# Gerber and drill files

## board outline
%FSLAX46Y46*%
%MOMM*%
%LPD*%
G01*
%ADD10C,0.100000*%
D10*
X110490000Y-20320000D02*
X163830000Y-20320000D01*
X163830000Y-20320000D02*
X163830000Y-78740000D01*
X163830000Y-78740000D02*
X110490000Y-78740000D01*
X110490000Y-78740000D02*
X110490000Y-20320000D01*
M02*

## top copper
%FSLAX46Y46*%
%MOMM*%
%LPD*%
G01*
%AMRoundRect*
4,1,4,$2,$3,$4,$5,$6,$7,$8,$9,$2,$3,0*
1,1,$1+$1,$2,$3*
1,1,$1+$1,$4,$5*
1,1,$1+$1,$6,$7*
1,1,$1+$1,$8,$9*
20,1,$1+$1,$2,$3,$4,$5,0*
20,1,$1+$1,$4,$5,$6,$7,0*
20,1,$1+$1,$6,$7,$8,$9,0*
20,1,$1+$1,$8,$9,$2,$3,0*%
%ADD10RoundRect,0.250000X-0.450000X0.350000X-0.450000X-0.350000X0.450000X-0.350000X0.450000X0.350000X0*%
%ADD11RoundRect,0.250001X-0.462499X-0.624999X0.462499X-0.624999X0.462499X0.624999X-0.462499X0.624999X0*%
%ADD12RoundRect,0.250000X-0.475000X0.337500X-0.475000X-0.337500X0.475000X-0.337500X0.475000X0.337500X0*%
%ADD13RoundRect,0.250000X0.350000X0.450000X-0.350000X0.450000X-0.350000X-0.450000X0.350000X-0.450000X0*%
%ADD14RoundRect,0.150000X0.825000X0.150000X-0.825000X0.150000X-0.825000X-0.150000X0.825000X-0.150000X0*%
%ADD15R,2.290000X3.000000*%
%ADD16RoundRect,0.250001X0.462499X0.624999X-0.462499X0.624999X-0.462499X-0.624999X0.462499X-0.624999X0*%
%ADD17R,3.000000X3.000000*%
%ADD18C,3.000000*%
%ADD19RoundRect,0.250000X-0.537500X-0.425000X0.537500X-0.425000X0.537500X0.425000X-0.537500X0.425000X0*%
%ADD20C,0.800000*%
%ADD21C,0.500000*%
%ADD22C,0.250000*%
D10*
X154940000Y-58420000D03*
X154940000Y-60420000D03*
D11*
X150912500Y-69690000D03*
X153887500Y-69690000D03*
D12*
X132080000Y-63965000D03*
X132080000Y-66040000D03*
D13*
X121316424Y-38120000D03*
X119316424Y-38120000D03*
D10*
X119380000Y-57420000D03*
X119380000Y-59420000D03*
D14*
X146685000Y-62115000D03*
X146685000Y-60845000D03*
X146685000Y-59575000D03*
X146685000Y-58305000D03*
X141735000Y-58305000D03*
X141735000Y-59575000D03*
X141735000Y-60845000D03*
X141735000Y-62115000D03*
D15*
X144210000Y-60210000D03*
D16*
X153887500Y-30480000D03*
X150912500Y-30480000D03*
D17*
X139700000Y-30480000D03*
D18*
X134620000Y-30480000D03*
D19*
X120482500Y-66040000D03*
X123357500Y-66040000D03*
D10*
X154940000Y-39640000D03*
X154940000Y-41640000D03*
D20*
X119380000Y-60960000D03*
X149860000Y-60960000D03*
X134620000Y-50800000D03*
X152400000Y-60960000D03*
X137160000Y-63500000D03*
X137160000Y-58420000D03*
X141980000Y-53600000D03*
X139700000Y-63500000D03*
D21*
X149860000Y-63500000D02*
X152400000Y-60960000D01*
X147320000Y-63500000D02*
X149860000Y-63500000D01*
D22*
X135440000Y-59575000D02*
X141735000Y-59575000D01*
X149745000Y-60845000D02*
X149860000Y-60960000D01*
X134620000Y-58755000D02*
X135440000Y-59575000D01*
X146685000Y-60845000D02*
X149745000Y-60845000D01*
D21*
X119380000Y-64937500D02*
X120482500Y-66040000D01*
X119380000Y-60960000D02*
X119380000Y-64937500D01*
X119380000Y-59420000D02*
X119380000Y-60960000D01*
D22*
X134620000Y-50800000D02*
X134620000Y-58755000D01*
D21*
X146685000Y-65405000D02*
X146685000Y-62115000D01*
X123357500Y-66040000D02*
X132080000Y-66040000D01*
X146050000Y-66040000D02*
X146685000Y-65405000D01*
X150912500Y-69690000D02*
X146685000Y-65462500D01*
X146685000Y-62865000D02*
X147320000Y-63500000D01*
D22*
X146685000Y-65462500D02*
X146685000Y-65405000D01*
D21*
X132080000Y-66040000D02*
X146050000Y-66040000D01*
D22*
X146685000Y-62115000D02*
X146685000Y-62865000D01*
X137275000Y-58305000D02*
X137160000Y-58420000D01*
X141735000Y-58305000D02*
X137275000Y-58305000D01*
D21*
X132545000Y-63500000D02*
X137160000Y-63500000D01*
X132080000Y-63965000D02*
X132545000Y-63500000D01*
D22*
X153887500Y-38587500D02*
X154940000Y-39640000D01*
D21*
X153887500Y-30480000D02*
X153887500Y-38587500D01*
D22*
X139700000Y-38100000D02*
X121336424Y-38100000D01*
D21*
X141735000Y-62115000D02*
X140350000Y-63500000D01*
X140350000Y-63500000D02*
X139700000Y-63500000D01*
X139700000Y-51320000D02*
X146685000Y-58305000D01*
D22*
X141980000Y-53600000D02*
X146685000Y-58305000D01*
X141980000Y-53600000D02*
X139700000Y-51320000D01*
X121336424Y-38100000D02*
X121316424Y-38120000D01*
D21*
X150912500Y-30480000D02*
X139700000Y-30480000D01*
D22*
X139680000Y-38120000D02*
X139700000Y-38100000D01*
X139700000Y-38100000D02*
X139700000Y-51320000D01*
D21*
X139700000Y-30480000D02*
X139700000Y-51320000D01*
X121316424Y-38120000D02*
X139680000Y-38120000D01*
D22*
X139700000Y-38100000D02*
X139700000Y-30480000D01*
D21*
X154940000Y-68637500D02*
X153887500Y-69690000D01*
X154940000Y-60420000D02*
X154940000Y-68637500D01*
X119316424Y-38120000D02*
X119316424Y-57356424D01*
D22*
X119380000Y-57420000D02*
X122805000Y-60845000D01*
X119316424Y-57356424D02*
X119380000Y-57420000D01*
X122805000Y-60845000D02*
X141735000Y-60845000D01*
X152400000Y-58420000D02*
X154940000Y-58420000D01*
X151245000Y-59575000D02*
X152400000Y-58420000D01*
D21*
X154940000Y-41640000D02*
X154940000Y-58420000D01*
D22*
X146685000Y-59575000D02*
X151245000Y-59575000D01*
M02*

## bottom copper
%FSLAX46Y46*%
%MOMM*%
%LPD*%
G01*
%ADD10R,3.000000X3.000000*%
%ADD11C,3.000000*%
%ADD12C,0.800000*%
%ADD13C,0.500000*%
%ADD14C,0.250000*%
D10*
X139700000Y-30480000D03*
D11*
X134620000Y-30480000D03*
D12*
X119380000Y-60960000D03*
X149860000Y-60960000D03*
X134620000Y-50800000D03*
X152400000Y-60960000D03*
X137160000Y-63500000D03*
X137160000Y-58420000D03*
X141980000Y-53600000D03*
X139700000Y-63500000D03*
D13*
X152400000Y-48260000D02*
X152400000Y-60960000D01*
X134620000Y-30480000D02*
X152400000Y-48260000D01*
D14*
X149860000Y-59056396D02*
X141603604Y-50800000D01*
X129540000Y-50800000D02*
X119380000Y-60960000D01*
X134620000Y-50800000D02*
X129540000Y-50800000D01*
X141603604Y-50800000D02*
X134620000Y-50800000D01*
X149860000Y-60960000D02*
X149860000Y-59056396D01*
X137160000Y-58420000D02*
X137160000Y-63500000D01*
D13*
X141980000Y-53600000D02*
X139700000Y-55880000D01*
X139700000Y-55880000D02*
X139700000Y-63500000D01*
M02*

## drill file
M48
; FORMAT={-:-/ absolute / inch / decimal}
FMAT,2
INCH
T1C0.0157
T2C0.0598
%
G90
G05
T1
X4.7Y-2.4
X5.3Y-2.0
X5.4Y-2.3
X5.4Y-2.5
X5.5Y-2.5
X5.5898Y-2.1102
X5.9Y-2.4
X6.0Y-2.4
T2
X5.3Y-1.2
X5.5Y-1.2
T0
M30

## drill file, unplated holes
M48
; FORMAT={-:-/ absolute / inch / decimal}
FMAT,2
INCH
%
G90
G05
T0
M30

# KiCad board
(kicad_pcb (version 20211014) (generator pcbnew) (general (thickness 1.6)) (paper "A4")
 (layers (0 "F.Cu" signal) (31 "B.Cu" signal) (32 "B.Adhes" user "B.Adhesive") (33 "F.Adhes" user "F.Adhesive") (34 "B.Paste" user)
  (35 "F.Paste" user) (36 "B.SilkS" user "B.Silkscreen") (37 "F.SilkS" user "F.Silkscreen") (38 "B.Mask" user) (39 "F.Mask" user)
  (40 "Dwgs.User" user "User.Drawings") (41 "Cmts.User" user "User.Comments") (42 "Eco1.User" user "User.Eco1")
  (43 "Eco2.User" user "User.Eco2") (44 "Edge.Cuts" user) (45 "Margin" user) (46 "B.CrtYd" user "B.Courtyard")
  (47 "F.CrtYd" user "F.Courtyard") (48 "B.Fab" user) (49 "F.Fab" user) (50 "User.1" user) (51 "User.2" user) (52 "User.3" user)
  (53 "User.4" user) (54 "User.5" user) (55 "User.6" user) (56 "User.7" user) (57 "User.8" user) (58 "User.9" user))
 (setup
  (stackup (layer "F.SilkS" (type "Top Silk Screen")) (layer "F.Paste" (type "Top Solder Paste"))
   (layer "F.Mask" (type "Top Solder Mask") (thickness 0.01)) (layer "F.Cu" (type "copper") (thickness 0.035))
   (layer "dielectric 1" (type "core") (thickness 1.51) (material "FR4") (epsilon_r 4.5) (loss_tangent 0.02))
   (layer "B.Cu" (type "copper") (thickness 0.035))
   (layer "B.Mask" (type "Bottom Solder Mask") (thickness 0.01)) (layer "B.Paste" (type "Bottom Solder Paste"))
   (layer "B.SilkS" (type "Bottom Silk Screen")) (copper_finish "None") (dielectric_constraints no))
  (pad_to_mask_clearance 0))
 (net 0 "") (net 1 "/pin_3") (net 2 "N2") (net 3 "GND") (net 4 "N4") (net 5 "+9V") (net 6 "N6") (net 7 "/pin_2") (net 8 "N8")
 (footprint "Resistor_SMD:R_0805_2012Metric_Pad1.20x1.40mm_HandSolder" (layer "F.Cu") (at 154.94 59.42 -90)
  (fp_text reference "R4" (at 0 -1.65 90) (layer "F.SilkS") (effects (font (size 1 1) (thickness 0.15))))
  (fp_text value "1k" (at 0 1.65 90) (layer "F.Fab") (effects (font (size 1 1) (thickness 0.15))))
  (pad "1" smd roundrect (at -1 0 270) (size 1.2 1.4) (layers "F.Cu" "F.Paste" "F.Mask") (roundrect_rratio 0.2083333333) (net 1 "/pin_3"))
  (pad "2" smd roundrect (at 1 0 270) (size 1.2 1.4) (layers "F.Cu" "F.Paste" "F.Mask") (roundrect_rratio 0.2083333333) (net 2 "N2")))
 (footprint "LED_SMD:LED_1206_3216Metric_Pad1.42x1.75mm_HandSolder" (layer "F.Cu") (at 152.4 69.69)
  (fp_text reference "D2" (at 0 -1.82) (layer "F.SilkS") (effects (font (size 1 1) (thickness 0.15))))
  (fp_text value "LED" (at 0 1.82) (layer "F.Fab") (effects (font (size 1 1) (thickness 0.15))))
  (pad "1" smd roundrect (at -1.4875 0) (size 1.425 1.75) (layers "F.Cu" "F.Paste" "F.Mask") (roundrect_rratio 0.1754392982) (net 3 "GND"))
  (pad "2" smd roundrect (at 1.4875 0) (size 1.425 1.75) (layers "F.Cu" "F.Paste" "F.Mask") (roundrect_rratio 0.1754392982) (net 2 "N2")))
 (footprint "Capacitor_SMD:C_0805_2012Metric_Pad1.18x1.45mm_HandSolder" (layer "F.Cu") (at 132.08 65.0025 -90)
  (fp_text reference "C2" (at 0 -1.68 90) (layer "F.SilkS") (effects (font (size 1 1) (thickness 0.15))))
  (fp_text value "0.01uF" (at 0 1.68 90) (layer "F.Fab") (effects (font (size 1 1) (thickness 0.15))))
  (pad "1" smd roundrect (at -1.0375 0 270) (size 1.175 1.45) (layers "F.Cu" "F.Paste" "F.Mask") (roundrect_rratio 0.2127659574)
   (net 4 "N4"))
  (pad "2" smd roundrect (at 1.0375 0 270) (size 1.175 1.45) (layers "F.Cu" "F.Paste" "F.Mask") (roundrect_rratio 0.2127659574)
   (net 3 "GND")))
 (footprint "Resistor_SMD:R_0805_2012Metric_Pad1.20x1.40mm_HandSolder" (layer "F.Cu") (at 120.316424 38.12 180)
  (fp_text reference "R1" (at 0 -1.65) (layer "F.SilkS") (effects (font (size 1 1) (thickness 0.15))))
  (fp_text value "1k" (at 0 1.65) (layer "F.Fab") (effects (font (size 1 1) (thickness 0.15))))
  (pad "1" smd roundrect (at -1 0 180) (size 1.2 1.4) (layers "F.Cu" "F.Paste" "F.Mask") (roundrect_rratio 0.2083333333) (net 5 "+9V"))
  (pad "2" smd roundrect (at 1 0 180) (size 1.2 1.4) (layers "F.Cu" "F.Paste" "F.Mask") (roundrect_rratio 0.2083333333) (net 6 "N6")))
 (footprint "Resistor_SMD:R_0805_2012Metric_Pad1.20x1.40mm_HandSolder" (layer "F.Cu") (at 119.38 58.42 -90)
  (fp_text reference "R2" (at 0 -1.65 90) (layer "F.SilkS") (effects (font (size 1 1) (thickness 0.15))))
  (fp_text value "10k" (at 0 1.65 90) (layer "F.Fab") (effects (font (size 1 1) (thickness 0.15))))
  (pad "1" smd roundrect (at -1 0 270) (size 1.2 1.4) (layers "F.Cu" "F.Paste" "F.Mask") (roundrect_rratio 0.2083333333) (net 6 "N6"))
  (pad "2" smd roundrect (at 1 0 270) (size 1.2 1.4) (layers "F.Cu" "F.Paste" "F.Mask") (roundrect_rratio 0.2083333333) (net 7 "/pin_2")))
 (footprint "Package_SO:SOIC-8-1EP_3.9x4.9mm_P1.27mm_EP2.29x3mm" (layer "F.Cu") (at 144.21 60.21 180)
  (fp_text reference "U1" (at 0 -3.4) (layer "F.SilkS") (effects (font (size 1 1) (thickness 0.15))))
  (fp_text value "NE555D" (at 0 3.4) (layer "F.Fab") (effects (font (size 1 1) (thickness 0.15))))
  (pad "" smd roundrect (at 0.57 0.75 180) (size 0.92 1.21) (layers "F.Paste") (roundrect_rratio 0.25))
  (pad "" smd roundrect (at -0.57 -0.75 180) (size 0.92 1.21) (layers "F.Paste") (roundrect_rratio 0.25))
  (pad "" smd roundrect (at 0.57 -0.75 180) (size 0.92 1.21) (layers "F.Paste") (roundrect_rratio 0.25))
  (pad "" smd roundrect (at -0.57 0.75 180) (size 0.92 1.21) (layers "F.Paste") (roundrect_rratio 0.25))
  (pad "1" smd roundrect (at -2.475 -1.905 180) (size 1.95 0.6) (layers "F.Cu" "F.Paste" "F.Mask") (roundrect_rratio 0.25) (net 3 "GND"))
  (pad "2" smd roundrect (at -2.475 -0.635 180) (size 1.95 0.6) (layers "F.Cu" "F.Paste" "F.Mask") (roundrect_rratio 0.25) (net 7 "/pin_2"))
  (pad "3" smd roundrect (at -2.475 0.635 180) (size 1.95 0.6) (layers "F.Cu" "F.Paste" "F.Mask") (roundrect_rratio 0.25) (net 1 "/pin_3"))
  (pad "4" smd roundrect (at -2.475 1.905 180) (size 1.95 0.6) (layers "F.Cu" "F.Paste" "F.Mask") (roundrect_rratio 0.25) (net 5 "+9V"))
  (pad "5" smd roundrect (at 2.475 1.905 180) (size 1.95 0.6) (layers "F.Cu" "F.Paste" "F.Mask") (roundrect_rratio 0.25) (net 4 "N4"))
  (pad "6" smd roundrect (at 2.475 0.635 180) (size 1.95 0.6) (layers "F.Cu" "F.Paste" "F.Mask") (roundrect_rratio 0.25) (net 7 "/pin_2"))
  (pad "7" smd roundrect (at 2.475 -0.635 180) (size 1.95 0.6) (layers "F.Cu" "F.Paste" "F.Mask") (roundrect_rratio 0.25) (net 6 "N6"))
  (pad "8" smd roundrect (at 2.475 -1.905 180) (size 1.95 0.6) (layers "F.Cu" "F.Paste" "F.Mask") (roundrect_rratio 0.25) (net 5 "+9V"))
  (pad "9" smd rect (at 0 0 180) (size 2.29 3) (layers "F.Cu" "F.Mask")))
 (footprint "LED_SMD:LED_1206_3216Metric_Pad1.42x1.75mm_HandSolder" (layer "F.Cu") (at 152.4 30.48 180)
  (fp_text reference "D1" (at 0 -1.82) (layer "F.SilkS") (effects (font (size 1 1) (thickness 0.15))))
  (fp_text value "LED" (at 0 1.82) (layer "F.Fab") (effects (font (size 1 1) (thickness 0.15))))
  (pad "1" smd roundrect (at -1.4875 0 180) (size 1.425 1.75) (layers "F.Cu" "F.Paste" "F.Mask") (roundrect_rratio 0.1754392982)
   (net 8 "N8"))
  (pad "2" smd roundrect (at 1.4875 0 180) (size 1.425 1.75) (layers "F.Cu" "F.Paste" "F.Mask") (roundrect_rratio 0.1754392982)
   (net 5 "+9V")))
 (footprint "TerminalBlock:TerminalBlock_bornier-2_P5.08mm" (layer "F.Cu") (at 139.7 30.48 180)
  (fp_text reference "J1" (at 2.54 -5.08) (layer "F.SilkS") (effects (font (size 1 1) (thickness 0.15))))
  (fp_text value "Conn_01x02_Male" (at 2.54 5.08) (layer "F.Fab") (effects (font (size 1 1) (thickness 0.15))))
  (pad "1" thru_hole rect (at 0 0 180) (size 3 3) (drill 1.52) (layers *.Cu *.Mask) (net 5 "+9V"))
  (pad "2" thru_hole circle (at 5.08 0 180) (size 3 3) (drill 1.52) (layers *.Cu *.Mask) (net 3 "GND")))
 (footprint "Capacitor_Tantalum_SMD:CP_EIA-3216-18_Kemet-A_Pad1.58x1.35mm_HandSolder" (layer "F.Cu") (at 121.92 66.04)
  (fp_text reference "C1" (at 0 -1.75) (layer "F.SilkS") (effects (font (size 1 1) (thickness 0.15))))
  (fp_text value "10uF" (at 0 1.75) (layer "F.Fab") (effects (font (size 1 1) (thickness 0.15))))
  (pad "1" smd roundrect (at -1.4375 0) (size 1.575 1.35) (layers "F.Cu" "F.Paste" "F.Mask") (roundrect_rratio 0.1851851852)
   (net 7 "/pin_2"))
  (pad "2" smd roundrect (at 1.4375 0) (size 1.575 1.35) (layers "F.Cu" "F.Paste" "F.Mask") (roundrect_rratio 0.1851851852) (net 3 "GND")))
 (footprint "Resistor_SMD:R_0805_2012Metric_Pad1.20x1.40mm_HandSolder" (layer "F.Cu") (at 154.94 40.64 -90)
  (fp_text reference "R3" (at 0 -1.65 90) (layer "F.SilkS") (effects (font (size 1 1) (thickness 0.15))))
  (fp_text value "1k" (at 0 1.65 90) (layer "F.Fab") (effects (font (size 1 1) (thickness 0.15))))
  (pad "1" smd roundrect (at -1 0 270) (size 1.2 1.4) (layers "F.Cu" "F.Paste" "F.Mask") (roundrect_rratio 0.2083333333) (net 8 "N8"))
  (pad "2" smd roundrect (at 1 0 270) (size 1.2 1.4) (layers "F.Cu" "F.Paste" "F.Mask") (roundrect_rratio 0.2083333333) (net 1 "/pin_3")))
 (gr_rect (start 110.49 20.32) (end 163.83 78.74) (layer "Edge.Cuts") (width 0.1) (fill none))
 (segment (start 135.44 59.575) (end 141.735 59.575) (width 0.25) (layer "F.Cu") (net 7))
 (segment (start 149.745 60.845) (end 149.86 60.96) (width 0.25) (layer "F.Cu") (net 7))
 (segment (start 134.62 58.755) (end 135.44 59.575) (width 0.25) (layer "F.Cu") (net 7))
 (segment (start 146.685 60.845) (end 149.745 60.845) (width 0.25) (layer "F.Cu") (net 7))
 (segment (start 119.38 64.9375) (end 120.4825 66.04) (width 0.5) (layer "F.Cu") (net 7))
 (segment (start 119.38 60.96) (end 119.38 64.9375) (width 0.5) (layer "F.Cu") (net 7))
 (segment (start 119.38 59.42) (end 119.38 60.96) (width 0.5) (layer "F.Cu") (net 7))
 (segment (start 134.62 50.8) (end 134.62 58.755) (width 0.25) (layer "F.Cu") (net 7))
 (via (at 119.38 60.96) (size 0.8) (drill 0.4) (layers "F.Cu" "B.Cu") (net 7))
 (via (at 149.86 60.96) (size 0.8) (drill 0.4) (layers "F.Cu" "B.Cu") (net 7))
 (via (at 134.62 50.8) (size 0.8) (drill 0.4) (layers "F.Cu" "B.Cu") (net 7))
 (segment (start 149.86 59.056396) (end 141.603604 50.8) (width 0.25) (layer "B.Cu") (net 7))
 (segment (start 129.54 50.8) (end 119.38 60.96) (width 0.25) (layer "B.Cu") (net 7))
 (segment (start 134.62 50.8) (end 129.54 50.8) (width 0.25) (layer "B.Cu") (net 7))
 (segment (start 141.603604 50.8) (end 134.62 50.8) (width 0.25) (layer "B.Cu") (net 7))
 (segment (start 149.86 60.96) (end 149.86 59.056396) (width 0.25) (layer "B.Cu") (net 7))
 (segment (start 146.685 65.405) (end 146.685 62.115) (width 0.5) (layer "F.Cu") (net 3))
 (segment (start 123.3575 66.04) (end 132.08 66.04) (width 0.5) (layer "F.Cu") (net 3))
 (segment (start 146.05 66.04) (end 146.685 65.405) (width 0.5) (layer "F.Cu") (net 3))
 (segment (start 150.9125 69.69) (end 146.685 65.4625) (width 0.5) (layer "F.Cu") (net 3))
 (segment (start 147.32 63.5) (end 149.86 63.5) (width 0.5) (layer "F.Cu") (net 3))
 (segment (start 149.86 63.5) (end 152.4 60.96) (width 0.5) (layer "F.Cu") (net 3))
 (segment (start 146.685 62.865) (end 147.32 63.5) (width 0.5) (layer "F.Cu") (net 3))
 (segment (start 146.685 65.4625) (end 146.685 65.405) (width 0.25) (layer "F.Cu") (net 3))
 (segment (start 132.08 66.04) (end 146.05 66.04) (width 0.5) (layer "F.Cu") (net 3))
 (segment (start 146.685 62.115) (end 146.685 62.865) (width 0.25) (layer "F.Cu") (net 3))
 (via (at 152.4 60.96) (size 0.8) (drill 0.4) (layers "F.Cu" "B.Cu") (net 3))
 (segment (start 152.4 48.26) (end 152.4 60.96) (width 0.5) (layer "B.Cu") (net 3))
 (segment (start 134.62 30.48) (end 152.4 48.26) (width 0.5) (layer "B.Cu") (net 3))
 (segment (start 137.275 58.305) (end 137.16 58.42) (width 0.25) (layer "F.Cu") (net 4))
 (segment (start 141.735 58.305) (end 137.275 58.305) (width 0.25) (layer "F.Cu") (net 4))
 (segment (start 132.545 63.5) (end 137.16 63.5) (width 0.5) (layer "F.Cu") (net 4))
 (segment (start 132.08 63.965) (end 132.545 63.5) (width 0.5) (layer "F.Cu") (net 4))
 (via (at 137.16 63.5) (size 0.8) (drill 0.4) (layers "F.Cu" "B.Cu") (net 4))
 (via (at 137.16 58.42) (size 0.8) (drill 0.4) (layers "F.Cu" "B.Cu") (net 4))
 (segment (start 137.16 58.42) (end 137.16 63.5) (width 0.25) (layer "B.Cu") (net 4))
 (segment (start 153.8875 38.5875) (end 154.94 39.64) (width 0.25) (layer "F.Cu") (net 8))
 (segment (start 153.8875 30.48) (end 153.8875 38.5875) (width 0.5) (layer "F.Cu") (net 8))
 (segment (start 139.7 38.1) (end 121.336424 38.1) (width 0.25) (layer "F.Cu") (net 5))
 (segment (start 141.735 62.115) (end 140.35 63.5) (width 0.5) (layer "F.Cu") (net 5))
 (segment (start 140.35 63.5) (end 139.7 63.5) (width 0.5) (layer "F.Cu") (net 5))
 (segment (start 139.7 51.32) (end 146.685 58.305) (width 0.5) (layer "F.Cu") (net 5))
 (segment (start 141.98 53.6) (end 146.685 58.305) (width 0.25) (layer "F.Cu") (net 5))
 (segment (start 141.98 53.6) (end 139.7 51.32) (width 0.25) (layer "F.Cu") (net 5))
 (segment (start 121.336424 38.1) (end 121.316424 38.12) (width 0.25) (layer "F.Cu") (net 5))
 (segment (start 150.9125 30.48) (end 139.7 30.48) (width 0.5) (layer "F.Cu") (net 5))
 (segment (start 139.68 38.12) (end 139.7 38.1) (width 0.25) (layer "F.Cu") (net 5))
 (segment (start 139.7 38.1) (end 139.7 51.32) (width 0.25) (layer "F.Cu") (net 5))
 (segment (start 139.7 30.48) (end 139.7 51.32) (width 0.5) (layer "F.Cu") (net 5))
 (segment (start 121.316424 38.12) (end 139.68 38.12) (width 0.5) (layer "F.Cu") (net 5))
 (segment (start 139.7 38.1) (end 139.7 30.48) (width 0.25) (layer "F.Cu") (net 5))
 (via (at 141.98 53.6) (size 0.8) (drill 0.4) (layers "F.Cu" "B.Cu") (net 5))
 (via (at 139.7 63.5) (size 0.8) (drill 0.4) (layers "F.Cu" "B.Cu") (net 5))
 (segment (start 141.98 53.6) (end 139.7 55.88) (width 0.5) (layer "B.Cu") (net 5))
 (segment (start 139.7 55.88) (end 139.7 63.5) (width 0.5) (layer "B.Cu") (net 5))
 (segment (start 154.94 68.6375) (end 153.8875 69.69) (width 0.5) (layer "F.Cu") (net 2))
 (segment (start 154.94 60.42) (end 154.94 68.6375) (width 0.5) (layer "F.Cu") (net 2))
 (segment (start 119.316424 38.12) (end 119.316424 57.356424) (width 0.5) (layer "F.Cu") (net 6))
 (segment (start 119.38 57.42) (end 122.805 60.845) (width 0.25) (layer "F.Cu") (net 6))
 (segment (start 119.316424 57.356424) (end 119.38 57.42) (width 0.25) (layer "F.Cu") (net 6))
 (segment (start 122.805 60.845) (end 141.735 60.845) (width 0.25) (layer "F.Cu") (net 6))
 (segment (start 152.4 58.42) (end 154.94 58.42) (width 0.25) (layer "F.Cu") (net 1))
 (segment (start 151.245 59.575) (end 152.4 58.42) (width 0.25) (layer "F.Cu") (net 1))
 (segment (start 154.94 41.64) (end 154.94 58.42) (width 0.5) (layer "F.Cu") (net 1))
 (segment (start 146.685 59.575) (end 151.245 59.575) (width 0.25) (layer "F.Cu") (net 1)))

